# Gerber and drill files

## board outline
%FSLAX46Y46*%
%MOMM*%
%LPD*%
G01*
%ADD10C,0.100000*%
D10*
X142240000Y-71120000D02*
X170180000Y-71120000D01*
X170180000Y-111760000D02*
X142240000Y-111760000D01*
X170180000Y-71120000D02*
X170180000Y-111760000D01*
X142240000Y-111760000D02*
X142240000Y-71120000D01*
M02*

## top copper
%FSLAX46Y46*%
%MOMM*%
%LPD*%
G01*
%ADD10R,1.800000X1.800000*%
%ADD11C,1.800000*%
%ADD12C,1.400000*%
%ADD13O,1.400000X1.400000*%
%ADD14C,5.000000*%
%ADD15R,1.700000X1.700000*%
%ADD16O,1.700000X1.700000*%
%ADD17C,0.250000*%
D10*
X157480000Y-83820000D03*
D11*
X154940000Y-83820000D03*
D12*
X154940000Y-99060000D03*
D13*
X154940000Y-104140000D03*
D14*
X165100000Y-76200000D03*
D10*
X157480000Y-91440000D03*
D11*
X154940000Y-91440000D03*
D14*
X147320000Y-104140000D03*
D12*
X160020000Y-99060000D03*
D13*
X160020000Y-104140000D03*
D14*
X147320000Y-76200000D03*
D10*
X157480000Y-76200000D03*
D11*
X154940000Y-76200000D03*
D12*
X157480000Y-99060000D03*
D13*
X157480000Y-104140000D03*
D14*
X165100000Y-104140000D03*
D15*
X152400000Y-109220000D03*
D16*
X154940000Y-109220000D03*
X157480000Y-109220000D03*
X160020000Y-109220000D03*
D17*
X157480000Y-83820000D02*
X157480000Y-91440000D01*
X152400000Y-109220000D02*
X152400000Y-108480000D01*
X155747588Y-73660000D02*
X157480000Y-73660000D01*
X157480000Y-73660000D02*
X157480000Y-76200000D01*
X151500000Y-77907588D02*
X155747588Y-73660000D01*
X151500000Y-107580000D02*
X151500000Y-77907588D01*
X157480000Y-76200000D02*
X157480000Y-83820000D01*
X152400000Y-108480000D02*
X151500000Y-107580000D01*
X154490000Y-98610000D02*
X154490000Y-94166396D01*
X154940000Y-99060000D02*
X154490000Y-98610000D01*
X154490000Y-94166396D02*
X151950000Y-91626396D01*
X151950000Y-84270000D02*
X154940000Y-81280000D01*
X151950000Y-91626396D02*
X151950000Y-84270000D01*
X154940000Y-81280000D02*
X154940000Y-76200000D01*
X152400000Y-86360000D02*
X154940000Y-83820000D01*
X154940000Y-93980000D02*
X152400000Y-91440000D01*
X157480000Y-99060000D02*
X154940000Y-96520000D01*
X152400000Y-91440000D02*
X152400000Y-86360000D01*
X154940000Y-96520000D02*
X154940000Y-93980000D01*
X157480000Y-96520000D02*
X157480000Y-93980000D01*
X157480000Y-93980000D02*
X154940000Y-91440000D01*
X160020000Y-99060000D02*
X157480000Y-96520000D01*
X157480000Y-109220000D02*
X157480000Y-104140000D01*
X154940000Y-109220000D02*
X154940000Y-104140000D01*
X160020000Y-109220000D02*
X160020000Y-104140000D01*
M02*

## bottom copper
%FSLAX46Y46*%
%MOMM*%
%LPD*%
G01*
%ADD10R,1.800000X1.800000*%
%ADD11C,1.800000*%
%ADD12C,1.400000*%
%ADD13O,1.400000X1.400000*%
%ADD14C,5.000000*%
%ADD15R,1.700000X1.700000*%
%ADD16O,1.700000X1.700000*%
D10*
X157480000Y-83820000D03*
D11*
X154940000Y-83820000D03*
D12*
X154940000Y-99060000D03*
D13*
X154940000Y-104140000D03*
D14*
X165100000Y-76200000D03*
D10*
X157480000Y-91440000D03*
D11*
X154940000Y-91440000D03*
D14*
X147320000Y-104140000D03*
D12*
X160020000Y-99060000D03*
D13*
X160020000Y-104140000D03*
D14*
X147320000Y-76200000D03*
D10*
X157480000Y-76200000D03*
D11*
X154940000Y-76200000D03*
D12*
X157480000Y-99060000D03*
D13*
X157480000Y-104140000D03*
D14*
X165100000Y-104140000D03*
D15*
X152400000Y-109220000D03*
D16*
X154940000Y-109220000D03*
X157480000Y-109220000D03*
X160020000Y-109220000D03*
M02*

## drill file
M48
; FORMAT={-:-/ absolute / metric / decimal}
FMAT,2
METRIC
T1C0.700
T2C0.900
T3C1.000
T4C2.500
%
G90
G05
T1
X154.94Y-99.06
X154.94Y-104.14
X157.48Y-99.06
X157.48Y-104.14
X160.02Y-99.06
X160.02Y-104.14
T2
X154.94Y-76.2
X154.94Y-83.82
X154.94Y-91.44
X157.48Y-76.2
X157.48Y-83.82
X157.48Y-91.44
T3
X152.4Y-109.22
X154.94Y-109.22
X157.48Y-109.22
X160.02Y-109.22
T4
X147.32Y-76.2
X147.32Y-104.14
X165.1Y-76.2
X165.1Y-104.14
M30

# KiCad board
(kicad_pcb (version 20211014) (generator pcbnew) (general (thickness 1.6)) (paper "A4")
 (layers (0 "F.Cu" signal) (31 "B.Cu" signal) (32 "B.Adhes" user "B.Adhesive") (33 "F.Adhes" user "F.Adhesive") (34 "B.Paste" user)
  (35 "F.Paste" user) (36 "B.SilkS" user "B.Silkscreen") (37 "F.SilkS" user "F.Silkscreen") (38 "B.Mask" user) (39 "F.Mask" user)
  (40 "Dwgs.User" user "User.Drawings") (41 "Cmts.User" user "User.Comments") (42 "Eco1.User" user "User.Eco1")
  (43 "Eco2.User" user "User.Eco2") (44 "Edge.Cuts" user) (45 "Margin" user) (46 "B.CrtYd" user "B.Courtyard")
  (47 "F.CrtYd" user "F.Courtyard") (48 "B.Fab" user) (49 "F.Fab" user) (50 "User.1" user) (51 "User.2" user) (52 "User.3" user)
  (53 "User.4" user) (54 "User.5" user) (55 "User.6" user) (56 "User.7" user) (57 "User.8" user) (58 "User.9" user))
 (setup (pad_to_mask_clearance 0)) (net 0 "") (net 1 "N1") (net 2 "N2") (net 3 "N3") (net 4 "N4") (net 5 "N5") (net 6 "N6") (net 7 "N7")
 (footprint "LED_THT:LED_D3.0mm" (layer "F.Cu") (at 157.48 83.82 180)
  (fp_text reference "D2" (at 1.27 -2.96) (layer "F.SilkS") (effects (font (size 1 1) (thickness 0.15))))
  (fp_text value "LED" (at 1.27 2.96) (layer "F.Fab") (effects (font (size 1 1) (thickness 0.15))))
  (pad "1" thru_hole rect (at 0 0 180) (size 1.8 1.8) (drill 0.9) (layers *.Cu *.Mask) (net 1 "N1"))
  (pad "2" thru_hole circle (at 2.54 0 180) (size 1.8 1.8) (drill 0.9) (layers *.Cu *.Mask) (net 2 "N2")))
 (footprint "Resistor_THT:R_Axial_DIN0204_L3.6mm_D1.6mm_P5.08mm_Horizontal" (layer "F.Cu") (at 154.94 99.06 -90)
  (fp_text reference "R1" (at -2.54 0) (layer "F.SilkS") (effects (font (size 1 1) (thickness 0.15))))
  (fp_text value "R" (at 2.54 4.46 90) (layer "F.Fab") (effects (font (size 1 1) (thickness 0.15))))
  (pad "1" thru_hole circle (at 0 0 270) (size 1.4 1.4) (drill 0.7) (layers *.Cu *.Mask) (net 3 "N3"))
  (pad "2" thru_hole oval (at 5.08 0 270) (size 1.4 1.4) (drill 0.7) (layers *.Cu *.Mask) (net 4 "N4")))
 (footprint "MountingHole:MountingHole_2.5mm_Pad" (layer "F.Cu") (at 165.1 76.2)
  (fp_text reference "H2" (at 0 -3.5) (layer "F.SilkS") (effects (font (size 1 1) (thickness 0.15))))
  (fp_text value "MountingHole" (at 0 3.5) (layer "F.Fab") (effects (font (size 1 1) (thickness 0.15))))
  (pad "1" thru_hole circle (at 0 0) (size 5 5) (drill 2.5) (layers *.Cu *.Mask)))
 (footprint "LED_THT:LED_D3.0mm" (layer "F.Cu") (at 157.48 91.44 180)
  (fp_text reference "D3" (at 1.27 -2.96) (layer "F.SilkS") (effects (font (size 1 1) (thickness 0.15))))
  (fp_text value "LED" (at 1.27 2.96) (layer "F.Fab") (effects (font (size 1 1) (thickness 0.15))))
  (pad "1" thru_hole rect (at 0 0 180) (size 1.8 1.8) (drill 0.9) (layers *.Cu *.Mask) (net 1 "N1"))
  (pad "2" thru_hole circle (at 2.54 0 180) (size 1.8 1.8) (drill 0.9) (layers *.Cu *.Mask) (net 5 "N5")))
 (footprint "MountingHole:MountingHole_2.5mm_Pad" (layer "F.Cu") (at 147.32 104.14)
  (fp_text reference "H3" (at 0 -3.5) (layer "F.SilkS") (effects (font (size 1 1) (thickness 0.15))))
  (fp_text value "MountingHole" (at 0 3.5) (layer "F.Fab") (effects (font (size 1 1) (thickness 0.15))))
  (pad "1" thru_hole circle (at 0 0) (size 5 5) (drill 2.5) (layers *.Cu *.Mask)))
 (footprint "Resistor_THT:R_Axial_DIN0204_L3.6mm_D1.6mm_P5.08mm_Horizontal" (layer "F.Cu") (at 160.02 99.06 -90)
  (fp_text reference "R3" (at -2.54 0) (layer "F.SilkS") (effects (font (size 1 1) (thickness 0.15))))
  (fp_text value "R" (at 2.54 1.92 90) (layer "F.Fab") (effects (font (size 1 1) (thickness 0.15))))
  (pad "1" thru_hole circle (at 0 0 270) (size 1.4 1.4) (drill 0.7) (layers *.Cu *.Mask) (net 5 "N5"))
  (pad "2" thru_hole oval (at 5.08 0 270) (size 1.4 1.4) (drill 0.7) (layers *.Cu *.Mask) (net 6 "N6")))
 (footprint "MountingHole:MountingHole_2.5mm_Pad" (layer "F.Cu") (at 147.32 76.2)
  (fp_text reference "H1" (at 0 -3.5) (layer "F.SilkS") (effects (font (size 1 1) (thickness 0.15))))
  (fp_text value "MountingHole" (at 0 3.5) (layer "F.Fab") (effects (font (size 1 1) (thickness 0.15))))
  (pad "1" thru_hole circle (at 0 0) (size 5 5) (drill 2.5) (layers *.Cu *.Mask)))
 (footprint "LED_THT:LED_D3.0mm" (layer "F.Cu") (at 157.48 76.2 180)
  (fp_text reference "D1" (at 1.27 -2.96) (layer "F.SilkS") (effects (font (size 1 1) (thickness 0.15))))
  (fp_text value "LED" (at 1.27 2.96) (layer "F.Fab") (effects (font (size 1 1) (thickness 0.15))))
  (pad "1" thru_hole rect (at 0 0 180) (size 1.8 1.8) (drill 0.9) (layers *.Cu *.Mask) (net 1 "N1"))
  (pad "2" thru_hole circle (at 2.54 0 180) (size 1.8 1.8) (drill 0.9) (layers *.Cu *.Mask) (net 3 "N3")))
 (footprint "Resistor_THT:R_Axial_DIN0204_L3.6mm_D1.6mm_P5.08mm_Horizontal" (layer "F.Cu") (at 157.48 99.06 -90)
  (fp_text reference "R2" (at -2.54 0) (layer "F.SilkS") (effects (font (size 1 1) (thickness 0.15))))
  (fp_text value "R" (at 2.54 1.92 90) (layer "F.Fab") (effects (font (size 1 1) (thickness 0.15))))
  (pad "1" thru_hole circle (at 0 0 270) (size 1.4 1.4) (drill 0.7) (layers *.Cu *.Mask) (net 2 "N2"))
  (pad "2" thru_hole oval (at 5.08 0 270) (size 1.4 1.4) (drill 0.7) (layers *.Cu *.Mask) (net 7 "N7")))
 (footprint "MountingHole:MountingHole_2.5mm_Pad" (layer "F.Cu") (at 165.1 104.14)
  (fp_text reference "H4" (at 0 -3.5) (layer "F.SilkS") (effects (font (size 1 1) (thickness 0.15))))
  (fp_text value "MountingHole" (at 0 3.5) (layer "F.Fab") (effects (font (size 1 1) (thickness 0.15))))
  (pad "1" thru_hole circle (at 0 0) (size 5 5) (drill 2.5) (layers *.Cu *.Mask)))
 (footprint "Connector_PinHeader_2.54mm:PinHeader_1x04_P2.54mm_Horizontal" (layer "B.Cu") (at 152.4 109.22 -90)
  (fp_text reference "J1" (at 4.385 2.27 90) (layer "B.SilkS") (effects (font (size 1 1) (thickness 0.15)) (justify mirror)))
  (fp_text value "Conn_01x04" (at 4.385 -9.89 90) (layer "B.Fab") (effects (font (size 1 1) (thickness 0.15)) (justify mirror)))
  (pad "1" thru_hole rect (at 0 0 270) (size 1.7 1.7) (drill 1) (layers *.Cu *.Mask) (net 1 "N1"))
  (pad "2" thru_hole oval (at 0 -2.54 270) (size 1.7 1.7) (drill 1) (layers *.Cu *.Mask) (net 4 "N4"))
  (pad "3" thru_hole oval (at 0 -5.08 270) (size 1.7 1.7) (drill 1) (layers *.Cu *.Mask) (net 7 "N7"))
  (pad "4" thru_hole oval (at 0 -7.62 270) (size 1.7 1.7) (drill 1) (layers *.Cu *.Mask) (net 6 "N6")))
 (gr_line (start 142.24 71.12) (end 170.18 71.12) (layer "Edge.Cuts") (width 0.1))
 (gr_line (start 170.18 111.76) (end 142.24 111.76) (layer "Edge.Cuts") (width 0.1))
 (gr_line (start 170.18 71.12) (end 170.18 111.76) (layer "Edge.Cuts") (width 0.1))
 (gr_line (start 142.24 111.76) (end 142.24 71.12) (layer "Edge.Cuts") (width 0.1))
 (segment (start 157.48 83.82) (end 157.48 91.44) (width 0.25) (layer "F.Cu") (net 1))
 (segment (start 152.4 109.22) (end 152.4 108.48) (width 0.25) (layer "F.Cu") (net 1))
 (segment (start 155.747588 73.66) (end 157.48 73.66) (width 0.25) (layer "F.Cu") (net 1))
 (segment (start 157.48 73.66) (end 157.48 76.2) (width 0.25) (layer "F.Cu") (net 1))
 (segment (start 151.5 77.907588) (end 155.747588 73.66) (width 0.25) (layer "F.Cu") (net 1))
 (segment (start 151.5 107.58) (end 151.5 77.907588) (width 0.25) (layer "F.Cu") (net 1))
 (segment (start 157.48 76.2) (end 157.48 83.82) (width 0.25) (layer "F.Cu") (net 1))
 (segment (start 152.4 108.48) (end 151.5 107.58) (width 0.25) (layer "F.Cu") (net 1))
 (segment (start 154.49 98.61) (end 154.49 94.166396) (width 0.25) (layer "F.Cu") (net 3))
 (segment (start 154.94 99.06) (end 154.49 98.61) (width 0.25) (layer "F.Cu") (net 3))
 (segment (start 154.49 94.166396) (end 151.95 91.626396) (width 0.25) (layer "F.Cu") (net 3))
 (segment (start 151.95 84.27) (end 154.94 81.28) (width 0.25) (layer "F.Cu") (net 3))
 (segment (start 151.95 91.626396) (end 151.95 84.27) (width 0.25) (layer "F.Cu") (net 3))
 (segment (start 154.94 81.28) (end 154.94 76.2) (width 0.25) (layer "F.Cu") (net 3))
 (segment (start 152.4 86.36) (end 154.94 83.82) (width 0.25) (layer "F.Cu") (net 2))
 (segment (start 154.94 93.98) (end 152.4 91.44) (width 0.25) (layer "F.Cu") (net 2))
 (segment (start 157.48 99.06) (end 154.94 96.52) (width 0.25) (layer "F.Cu") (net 2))
 (segment (start 152.4 91.44) (end 152.4 86.36) (width 0.25) (layer "F.Cu") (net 2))
 (segment (start 154.94 96.52) (end 154.94 93.98) (width 0.25) (layer "F.Cu") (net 2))
 (segment (start 157.48 96.52) (end 157.48 93.98) (width 0.25) (layer "F.Cu") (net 5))
 (segment (start 157.48 93.98) (end 154.94 91.44) (width 0.25) (layer "F.Cu") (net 5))
 (segment (start 160.02 99.06) (end 157.48 96.52) (width 0.25) (layer "F.Cu") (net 5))
 (segment (start 157.48 109.22) (end 157.48 104.14) (width 0.25) (layer "F.Cu") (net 7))
 (segment (start 154.94 109.22) (end 154.94 104.14) (width 0.25) (layer "F.Cu") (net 4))
 (segment (start 160.02 109.22) (end 160.02 104.14) (width 0.25) (layer "F.Cu") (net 6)))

